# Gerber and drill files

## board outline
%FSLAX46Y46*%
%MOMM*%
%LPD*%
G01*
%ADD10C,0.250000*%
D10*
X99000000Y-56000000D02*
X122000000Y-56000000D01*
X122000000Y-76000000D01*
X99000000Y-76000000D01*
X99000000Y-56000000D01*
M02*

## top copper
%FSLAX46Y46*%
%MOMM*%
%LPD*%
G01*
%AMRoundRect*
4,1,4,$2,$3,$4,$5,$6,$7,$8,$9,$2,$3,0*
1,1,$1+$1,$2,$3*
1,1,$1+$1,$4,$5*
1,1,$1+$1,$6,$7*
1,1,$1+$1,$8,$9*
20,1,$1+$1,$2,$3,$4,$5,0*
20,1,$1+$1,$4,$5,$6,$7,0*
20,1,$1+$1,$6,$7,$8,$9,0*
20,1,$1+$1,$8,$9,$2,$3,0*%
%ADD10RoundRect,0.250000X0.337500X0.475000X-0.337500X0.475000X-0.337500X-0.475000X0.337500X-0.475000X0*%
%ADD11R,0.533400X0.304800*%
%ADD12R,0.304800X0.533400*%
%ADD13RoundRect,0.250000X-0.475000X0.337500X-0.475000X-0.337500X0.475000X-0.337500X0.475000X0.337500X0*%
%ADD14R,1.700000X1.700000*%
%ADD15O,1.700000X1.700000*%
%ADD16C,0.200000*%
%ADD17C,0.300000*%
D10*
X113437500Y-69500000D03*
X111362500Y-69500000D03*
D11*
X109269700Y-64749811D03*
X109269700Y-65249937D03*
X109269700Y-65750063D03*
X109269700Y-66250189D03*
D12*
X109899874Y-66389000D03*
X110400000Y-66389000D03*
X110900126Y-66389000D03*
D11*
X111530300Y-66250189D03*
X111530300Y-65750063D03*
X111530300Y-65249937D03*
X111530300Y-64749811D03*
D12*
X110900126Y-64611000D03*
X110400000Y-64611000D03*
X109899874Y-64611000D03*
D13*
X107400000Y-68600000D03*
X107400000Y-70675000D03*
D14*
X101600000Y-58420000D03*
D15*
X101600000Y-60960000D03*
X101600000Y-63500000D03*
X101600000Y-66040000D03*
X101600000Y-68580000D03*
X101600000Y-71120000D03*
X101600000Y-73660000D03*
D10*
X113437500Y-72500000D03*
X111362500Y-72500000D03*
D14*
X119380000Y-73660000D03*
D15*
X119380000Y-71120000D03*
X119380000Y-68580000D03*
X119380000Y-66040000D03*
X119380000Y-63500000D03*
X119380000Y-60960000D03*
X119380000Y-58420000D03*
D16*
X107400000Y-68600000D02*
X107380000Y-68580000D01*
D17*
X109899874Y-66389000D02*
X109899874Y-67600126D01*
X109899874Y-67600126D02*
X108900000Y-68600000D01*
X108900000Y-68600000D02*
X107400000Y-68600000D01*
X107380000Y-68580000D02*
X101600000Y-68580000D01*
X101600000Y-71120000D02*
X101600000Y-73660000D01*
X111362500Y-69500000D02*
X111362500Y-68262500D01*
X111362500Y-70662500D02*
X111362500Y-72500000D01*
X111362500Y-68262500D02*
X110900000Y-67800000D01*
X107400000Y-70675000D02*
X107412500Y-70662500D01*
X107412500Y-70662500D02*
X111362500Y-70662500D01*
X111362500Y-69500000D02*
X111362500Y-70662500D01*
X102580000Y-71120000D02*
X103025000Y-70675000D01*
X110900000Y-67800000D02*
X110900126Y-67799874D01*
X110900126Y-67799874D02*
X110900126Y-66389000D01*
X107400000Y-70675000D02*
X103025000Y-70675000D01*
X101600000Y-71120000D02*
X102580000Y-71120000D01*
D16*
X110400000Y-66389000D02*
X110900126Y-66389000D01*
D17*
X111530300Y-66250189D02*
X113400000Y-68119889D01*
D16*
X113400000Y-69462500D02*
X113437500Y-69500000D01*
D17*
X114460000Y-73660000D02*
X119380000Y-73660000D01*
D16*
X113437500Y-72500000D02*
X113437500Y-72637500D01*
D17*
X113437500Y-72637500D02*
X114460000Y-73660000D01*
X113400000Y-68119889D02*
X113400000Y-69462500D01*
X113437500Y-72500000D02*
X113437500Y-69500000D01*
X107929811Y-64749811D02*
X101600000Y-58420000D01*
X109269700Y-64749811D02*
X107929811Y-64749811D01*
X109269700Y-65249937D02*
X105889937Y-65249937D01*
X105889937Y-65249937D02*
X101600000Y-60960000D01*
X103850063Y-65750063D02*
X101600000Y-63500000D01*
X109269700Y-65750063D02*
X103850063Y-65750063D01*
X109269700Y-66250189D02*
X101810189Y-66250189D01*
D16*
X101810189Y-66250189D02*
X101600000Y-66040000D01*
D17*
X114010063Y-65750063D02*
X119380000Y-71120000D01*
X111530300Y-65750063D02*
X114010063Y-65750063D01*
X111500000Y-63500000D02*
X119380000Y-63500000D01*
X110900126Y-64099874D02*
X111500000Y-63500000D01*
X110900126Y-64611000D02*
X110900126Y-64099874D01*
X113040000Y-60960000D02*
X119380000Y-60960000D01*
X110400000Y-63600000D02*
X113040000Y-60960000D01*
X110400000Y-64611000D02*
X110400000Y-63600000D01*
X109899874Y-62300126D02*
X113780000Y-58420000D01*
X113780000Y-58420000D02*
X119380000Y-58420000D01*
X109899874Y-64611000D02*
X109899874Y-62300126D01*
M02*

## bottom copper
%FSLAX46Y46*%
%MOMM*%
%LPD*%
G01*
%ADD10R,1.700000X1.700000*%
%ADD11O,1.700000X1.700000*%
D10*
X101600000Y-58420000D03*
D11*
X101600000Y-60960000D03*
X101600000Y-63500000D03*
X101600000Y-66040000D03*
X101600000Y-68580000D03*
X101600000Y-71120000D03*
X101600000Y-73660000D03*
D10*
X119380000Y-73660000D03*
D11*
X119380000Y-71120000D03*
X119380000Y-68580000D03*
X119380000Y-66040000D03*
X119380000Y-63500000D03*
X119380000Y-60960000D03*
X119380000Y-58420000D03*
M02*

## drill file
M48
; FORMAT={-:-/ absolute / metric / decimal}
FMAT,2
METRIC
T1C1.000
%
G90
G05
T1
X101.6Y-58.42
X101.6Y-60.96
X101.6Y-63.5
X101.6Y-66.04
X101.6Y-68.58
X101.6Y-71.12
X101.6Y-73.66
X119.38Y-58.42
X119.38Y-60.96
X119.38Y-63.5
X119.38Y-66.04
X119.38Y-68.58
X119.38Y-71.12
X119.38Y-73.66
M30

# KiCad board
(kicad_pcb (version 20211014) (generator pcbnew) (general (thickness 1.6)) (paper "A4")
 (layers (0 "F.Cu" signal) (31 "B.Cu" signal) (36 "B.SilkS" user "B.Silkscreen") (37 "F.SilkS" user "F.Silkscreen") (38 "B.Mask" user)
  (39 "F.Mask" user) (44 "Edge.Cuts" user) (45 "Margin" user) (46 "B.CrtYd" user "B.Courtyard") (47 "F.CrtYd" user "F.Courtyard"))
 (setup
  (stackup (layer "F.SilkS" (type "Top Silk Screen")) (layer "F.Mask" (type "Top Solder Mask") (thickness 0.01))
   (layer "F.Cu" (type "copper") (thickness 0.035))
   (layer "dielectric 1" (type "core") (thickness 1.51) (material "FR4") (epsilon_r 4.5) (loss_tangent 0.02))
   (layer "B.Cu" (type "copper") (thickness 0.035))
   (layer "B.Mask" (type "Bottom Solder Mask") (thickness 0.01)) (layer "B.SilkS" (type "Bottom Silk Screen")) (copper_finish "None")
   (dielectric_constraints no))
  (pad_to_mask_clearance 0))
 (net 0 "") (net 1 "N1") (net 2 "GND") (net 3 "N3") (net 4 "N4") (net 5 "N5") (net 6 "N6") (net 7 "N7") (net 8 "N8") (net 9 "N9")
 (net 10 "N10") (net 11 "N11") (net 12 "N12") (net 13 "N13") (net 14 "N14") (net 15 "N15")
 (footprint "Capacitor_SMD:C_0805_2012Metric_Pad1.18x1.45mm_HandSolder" (layer "F.Cu") (at 112.4 69.5 180)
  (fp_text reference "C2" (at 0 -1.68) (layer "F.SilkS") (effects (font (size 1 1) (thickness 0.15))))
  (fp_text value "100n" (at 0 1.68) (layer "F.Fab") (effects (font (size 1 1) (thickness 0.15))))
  (pad "1" smd roundrect (at -1.0375 0 180) (size 1.175 1.45) (layers "F.Cu" "F.Paste" "F.Mask") (roundrect_rratio 0.2127659574)
   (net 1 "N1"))
  (pad "2" smd roundrect (at 1.0375 0 180) (size 1.175 1.45) (layers "F.Cu" "F.Paste" "F.Mask") (roundrect_rratio 0.2127659574)
   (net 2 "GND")))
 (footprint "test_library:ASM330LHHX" (layer "F.Cu") (at 110.4 65.5)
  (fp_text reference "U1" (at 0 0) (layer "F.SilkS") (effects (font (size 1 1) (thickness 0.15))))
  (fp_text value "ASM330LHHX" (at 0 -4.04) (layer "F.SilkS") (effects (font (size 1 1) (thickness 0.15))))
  (pad "1" smd rect (at -1.1303 -0.750189 90) (size 0.3048 0.5334) (layers "F.Cu" "F.Paste" "F.Mask") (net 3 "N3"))
  (pad "2" smd rect (at -1.1303 -0.250063 90) (size 0.3048 0.5334) (layers "F.Cu" "F.Paste" "F.Mask") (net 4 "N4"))
  (pad "3" smd rect (at -1.1303 0.250063 90) (size 0.3048 0.5334) (layers "F.Cu" "F.Paste" "F.Mask") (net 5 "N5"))
  (pad "4" smd rect (at -1.1303 0.750189 90) (size 0.3048 0.5334) (layers "F.Cu" "F.Paste" "F.Mask") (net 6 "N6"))
  (pad "5" smd rect (at -0.500126 0.889) (size 0.3048 0.5334) (layers "F.Cu" "F.Paste" "F.Mask") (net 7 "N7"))
  (pad "6" smd rect (at 0 0.889) (size 0.3048 0.5334) (layers "F.Cu" "F.Paste" "F.Mask") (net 2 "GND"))
  (pad "7" smd rect (at 0.500126 0.889) (size 0.3048 0.5334) (layers "F.Cu" "F.Paste" "F.Mask") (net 2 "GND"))
  (pad "8" smd rect (at 1.1303 0.750189 90) (size 0.3048 0.5334) (layers "F.Cu" "F.Paste" "F.Mask") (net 1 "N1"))
  (pad "9" smd rect (at 1.1303 0.250063 90) (size 0.3048 0.5334) (layers "F.Cu" "F.Paste" "F.Mask") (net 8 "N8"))
  (pad "10" smd rect (at 1.1303 -0.250063 90) (size 0.3048 0.5334) (layers "F.Cu" "F.Paste" "F.Mask") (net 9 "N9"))
  (pad "11" smd rect (at 1.1303 -0.750189 90) (size 0.3048 0.5334) (layers "F.Cu" "F.Paste" "F.Mask") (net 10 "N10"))
  (pad "12" smd rect (at 0.500126 -0.889) (size 0.3048 0.5334) (layers "F.Cu" "F.Paste" "F.Mask") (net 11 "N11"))
  (pad "13" smd rect (at 0 -0.889) (size 0.3048 0.5334) (layers "F.Cu" "F.Paste" "F.Mask") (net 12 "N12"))
  (pad "14" smd rect (at -0.500126 -0.889) (size 0.3048 0.5334) (layers "F.Cu" "F.Paste" "F.Mask") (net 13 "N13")))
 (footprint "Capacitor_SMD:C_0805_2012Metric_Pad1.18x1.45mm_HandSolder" (layer "F.Cu") (at 107.4 69.6375 -90)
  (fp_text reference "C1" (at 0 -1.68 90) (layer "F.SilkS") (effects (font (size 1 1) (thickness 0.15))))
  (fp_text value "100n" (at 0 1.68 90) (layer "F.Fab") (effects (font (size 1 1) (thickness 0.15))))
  (pad "1" smd roundrect (at -1.0375 0 270) (size 1.175 1.45) (layers "F.Cu" "F.Paste" "F.Mask") (roundrect_rratio 0.2127659574)
   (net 7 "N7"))
  (pad "2" smd roundrect (at 1.0375 0 270) (size 1.175 1.45) (layers "F.Cu" "F.Paste" "F.Mask") (roundrect_rratio 0.2127659574)
   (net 2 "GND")))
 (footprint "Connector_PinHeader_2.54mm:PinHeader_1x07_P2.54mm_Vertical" (layer "F.Cu") (at 101.6 58.42)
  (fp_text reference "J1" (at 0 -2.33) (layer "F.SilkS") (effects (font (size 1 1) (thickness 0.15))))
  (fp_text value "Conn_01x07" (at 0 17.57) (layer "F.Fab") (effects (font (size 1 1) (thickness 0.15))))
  (pad "1" thru_hole rect (at 0 0) (size 1.7 1.7) (drill 1) (layers *.Cu *.Mask) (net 3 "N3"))
  (pad "2" thru_hole oval (at 0 2.54) (size 1.7 1.7) (drill 1) (layers *.Cu *.Mask) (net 4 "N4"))
  (pad "3" thru_hole oval (at 0 5.08) (size 1.7 1.7) (drill 1) (layers *.Cu *.Mask) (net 5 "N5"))
  (pad "4" thru_hole oval (at 0 7.62) (size 1.7 1.7) (drill 1) (layers *.Cu *.Mask) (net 6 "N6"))
  (pad "5" thru_hole oval (at 0 10.16) (size 1.7 1.7) (drill 1) (layers *.Cu *.Mask) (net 7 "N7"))
  (pad "6" thru_hole oval (at 0 12.7) (size 1.7 1.7) (drill 1) (layers *.Cu *.Mask) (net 2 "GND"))
  (pad "7" thru_hole oval (at 0 15.24) (size 1.7 1.7) (drill 1) (layers *.Cu *.Mask) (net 2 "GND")))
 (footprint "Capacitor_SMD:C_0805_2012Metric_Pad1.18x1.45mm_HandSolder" (layer "F.Cu") (at 112.4 72.5 180)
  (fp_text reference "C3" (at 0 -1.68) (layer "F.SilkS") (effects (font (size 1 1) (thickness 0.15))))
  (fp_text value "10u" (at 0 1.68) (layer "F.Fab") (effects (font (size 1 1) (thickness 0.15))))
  (pad "1" smd roundrect (at -1.0375 0 180) (size 1.175 1.45) (layers "F.Cu" "F.Paste" "F.Mask") (roundrect_rratio 0.2127659574)
   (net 1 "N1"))
  (pad "2" smd roundrect (at 1.0375 0 180) (size 1.175 1.45) (layers "F.Cu" "F.Paste" "F.Mask") (roundrect_rratio 0.2127659574)
   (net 2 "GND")))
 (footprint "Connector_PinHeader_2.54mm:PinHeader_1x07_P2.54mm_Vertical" (layer "F.Cu") (at 119.38 73.66 180)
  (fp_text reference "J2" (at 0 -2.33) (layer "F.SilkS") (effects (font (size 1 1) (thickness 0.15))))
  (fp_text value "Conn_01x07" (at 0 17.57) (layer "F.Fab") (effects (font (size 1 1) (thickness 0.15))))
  (pad "1" thru_hole rect (at 0 0 180) (size 1.7 1.7) (drill 1) (layers *.Cu *.Mask) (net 1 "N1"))
  (pad "2" thru_hole oval (at 0 2.54 180) (size 1.7 1.7) (drill 1) (layers *.Cu *.Mask) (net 8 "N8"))
  (pad "3" thru_hole oval (at 0 5.08 180) (size 1.7 1.7) (drill 1) (layers *.Cu *.Mask) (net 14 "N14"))
  (pad "4" thru_hole oval (at 0 7.62 180) (size 1.7 1.7) (drill 1) (layers *.Cu *.Mask) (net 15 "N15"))
  (pad "5" thru_hole oval (at 0 10.16 180) (size 1.7 1.7) (drill 1) (layers *.Cu *.Mask) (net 11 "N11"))
  (pad "6" thru_hole oval (at 0 12.7 180) (size 1.7 1.7) (drill 1) (layers *.Cu *.Mask) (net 12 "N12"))
  (pad "7" thru_hole oval (at 0 15.24 180) (size 1.7 1.7) (drill 1) (layers *.Cu *.Mask) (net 13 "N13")))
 (gr_rect (start 99 76) (end 122 56) (layer "Edge.Cuts") (width 0.25) (fill none))
 (segment (start 107.4 68.6) (end 107.38 68.58) (width 0.2) (layer "F.Cu") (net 7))
 (segment (start 109.899874 66.389) (end 109.899874 67.600126) (width 0.3) (layer "F.Cu") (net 7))
 (segment (start 109.899874 67.600126) (end 108.9 68.6) (width 0.3) (layer "F.Cu") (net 7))
 (segment (start 108.9 68.6) (end 107.4 68.6) (width 0.3) (layer "F.Cu") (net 7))
 (segment (start 107.38 68.58) (end 101.6 68.58) (width 0.3) (layer "F.Cu") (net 7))
 (segment (start 101.6 71.12) (end 101.6 73.66) (width 0.3) (layer "F.Cu") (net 2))
 (segment (start 111.3625 69.5) (end 111.3625 68.2625) (width 0.3) (layer "F.Cu") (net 2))
 (segment (start 111.3625 70.6625) (end 111.3625 72.5) (width 0.3) (layer "F.Cu") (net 2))
 (segment (start 111.3625 68.2625) (end 110.9 67.8) (width 0.3) (layer "F.Cu") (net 2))
 (segment (start 107.4 70.675) (end 107.4125 70.6625) (width 0.3) (layer "F.Cu") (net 2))
 (segment (start 107.4125 70.6625) (end 111.3625 70.6625) (width 0.3) (layer "F.Cu") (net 2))
 (segment (start 111.3625 69.5) (end 111.3625 70.6625) (width 0.3) (layer "F.Cu") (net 2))
 (segment (start 102.58 71.12) (end 103.025 70.675) (width 0.3) (layer "F.Cu") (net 2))
 (segment (start 110.9 67.8) (end 110.900126 67.799874) (width 0.3) (layer "F.Cu") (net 2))
 (segment (start 110.900126 67.799874) (end 110.900126 66.389) (width 0.3) (layer "F.Cu") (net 2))
 (segment (start 107.4 70.675) (end 103.025 70.675) (width 0.3) (layer "F.Cu") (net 2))
 (segment (start 101.6 71.12) (end 102.58 71.12) (width 0.3) (layer "F.Cu") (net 2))
 (segment (start 110.4 66.389) (end 110.900126 66.389) (width 0.2) (layer "F.Cu") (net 2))
 (segment (start 111.5303 66.250189) (end 113.4 68.119889) (width 0.3) (layer "F.Cu") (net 1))
 (segment (start 113.4 69.4625) (end 113.4375 69.5) (width 0.2) (layer "F.Cu") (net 1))
 (segment (start 114.46 73.66) (end 119.38 73.66) (width 0.3) (layer "F.Cu") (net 1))
 (segment (start 113.4375 72.5) (end 113.4375 72.6375) (width 0.2) (layer "F.Cu") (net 1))
 (segment (start 113.4375 72.6375) (end 114.46 73.66) (width 0.3) (layer "F.Cu") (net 1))
 (segment (start 113.4 68.119889) (end 113.4 69.4625) (width 0.3) (layer "F.Cu") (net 1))
 (segment (start 113.4375 72.5) (end 113.4375 69.5) (width 0.3) (layer "F.Cu") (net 1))
 (segment (start 107.929811 64.749811) (end 101.6 58.42) (width 0.3) (layer "F.Cu") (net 3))
 (segment (start 109.2697 64.749811) (end 107.929811 64.749811) (width 0.3) (layer "F.Cu") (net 3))
 (segment (start 109.2697 65.249937) (end 105.889937 65.249937) (width 0.3) (layer "F.Cu") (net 4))
 (segment (start 105.889937 65.249937) (end 101.6 60.96) (width 0.3) (layer "F.Cu") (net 4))
 (segment (start 103.850063 65.750063) (end 101.6 63.5) (width 0.3) (layer "F.Cu") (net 5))
 (segment (start 109.2697 65.750063) (end 103.850063 65.750063) (width 0.3) (layer "F.Cu") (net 5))
 (segment (start 109.2697 66.250189) (end 101.810189 66.250189) (width 0.3) (layer "F.Cu") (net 6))
 (segment (start 101.810189 66.250189) (end 101.6 66.04) (width 0.2) (layer "F.Cu") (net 6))
 (segment (start 114.010063 65.750063) (end 119.38 71.12) (width 0.3) (layer "F.Cu") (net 8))
 (segment (start 111.5303 65.750063) (end 114.010063 65.750063) (width 0.3) (layer "F.Cu") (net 8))
 (segment (start 111.5 63.5) (end 119.38 63.5) (width 0.3) (layer "F.Cu") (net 11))
 (segment (start 110.900126 64.099874) (end 111.5 63.5) (width 0.3) (layer "F.Cu") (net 11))
 (segment (start 110.900126 64.611) (end 110.900126 64.099874) (width 0.3) (layer "F.Cu") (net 11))
 (segment (start 113.04 60.96) (end 119.38 60.96) (width 0.3) (layer "F.Cu") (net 12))
 (segment (start 110.4 63.6) (end 113.04 60.96) (width 0.3) (layer "F.Cu") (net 12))
 (segment (start 110.4 64.611) (end 110.4 63.6) (width 0.3) (layer "F.Cu") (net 12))
 (segment (start 109.899874 62.300126) (end 113.78 58.42) (width 0.3) (layer "F.Cu") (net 13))
 (segment (start 113.78 58.42) (end 119.38 58.42) (width 0.3) (layer "F.Cu") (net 13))
 (segment (start 109.899874 64.611) (end 109.899874 62.300126) (width 0.3) (layer "F.Cu") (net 13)))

